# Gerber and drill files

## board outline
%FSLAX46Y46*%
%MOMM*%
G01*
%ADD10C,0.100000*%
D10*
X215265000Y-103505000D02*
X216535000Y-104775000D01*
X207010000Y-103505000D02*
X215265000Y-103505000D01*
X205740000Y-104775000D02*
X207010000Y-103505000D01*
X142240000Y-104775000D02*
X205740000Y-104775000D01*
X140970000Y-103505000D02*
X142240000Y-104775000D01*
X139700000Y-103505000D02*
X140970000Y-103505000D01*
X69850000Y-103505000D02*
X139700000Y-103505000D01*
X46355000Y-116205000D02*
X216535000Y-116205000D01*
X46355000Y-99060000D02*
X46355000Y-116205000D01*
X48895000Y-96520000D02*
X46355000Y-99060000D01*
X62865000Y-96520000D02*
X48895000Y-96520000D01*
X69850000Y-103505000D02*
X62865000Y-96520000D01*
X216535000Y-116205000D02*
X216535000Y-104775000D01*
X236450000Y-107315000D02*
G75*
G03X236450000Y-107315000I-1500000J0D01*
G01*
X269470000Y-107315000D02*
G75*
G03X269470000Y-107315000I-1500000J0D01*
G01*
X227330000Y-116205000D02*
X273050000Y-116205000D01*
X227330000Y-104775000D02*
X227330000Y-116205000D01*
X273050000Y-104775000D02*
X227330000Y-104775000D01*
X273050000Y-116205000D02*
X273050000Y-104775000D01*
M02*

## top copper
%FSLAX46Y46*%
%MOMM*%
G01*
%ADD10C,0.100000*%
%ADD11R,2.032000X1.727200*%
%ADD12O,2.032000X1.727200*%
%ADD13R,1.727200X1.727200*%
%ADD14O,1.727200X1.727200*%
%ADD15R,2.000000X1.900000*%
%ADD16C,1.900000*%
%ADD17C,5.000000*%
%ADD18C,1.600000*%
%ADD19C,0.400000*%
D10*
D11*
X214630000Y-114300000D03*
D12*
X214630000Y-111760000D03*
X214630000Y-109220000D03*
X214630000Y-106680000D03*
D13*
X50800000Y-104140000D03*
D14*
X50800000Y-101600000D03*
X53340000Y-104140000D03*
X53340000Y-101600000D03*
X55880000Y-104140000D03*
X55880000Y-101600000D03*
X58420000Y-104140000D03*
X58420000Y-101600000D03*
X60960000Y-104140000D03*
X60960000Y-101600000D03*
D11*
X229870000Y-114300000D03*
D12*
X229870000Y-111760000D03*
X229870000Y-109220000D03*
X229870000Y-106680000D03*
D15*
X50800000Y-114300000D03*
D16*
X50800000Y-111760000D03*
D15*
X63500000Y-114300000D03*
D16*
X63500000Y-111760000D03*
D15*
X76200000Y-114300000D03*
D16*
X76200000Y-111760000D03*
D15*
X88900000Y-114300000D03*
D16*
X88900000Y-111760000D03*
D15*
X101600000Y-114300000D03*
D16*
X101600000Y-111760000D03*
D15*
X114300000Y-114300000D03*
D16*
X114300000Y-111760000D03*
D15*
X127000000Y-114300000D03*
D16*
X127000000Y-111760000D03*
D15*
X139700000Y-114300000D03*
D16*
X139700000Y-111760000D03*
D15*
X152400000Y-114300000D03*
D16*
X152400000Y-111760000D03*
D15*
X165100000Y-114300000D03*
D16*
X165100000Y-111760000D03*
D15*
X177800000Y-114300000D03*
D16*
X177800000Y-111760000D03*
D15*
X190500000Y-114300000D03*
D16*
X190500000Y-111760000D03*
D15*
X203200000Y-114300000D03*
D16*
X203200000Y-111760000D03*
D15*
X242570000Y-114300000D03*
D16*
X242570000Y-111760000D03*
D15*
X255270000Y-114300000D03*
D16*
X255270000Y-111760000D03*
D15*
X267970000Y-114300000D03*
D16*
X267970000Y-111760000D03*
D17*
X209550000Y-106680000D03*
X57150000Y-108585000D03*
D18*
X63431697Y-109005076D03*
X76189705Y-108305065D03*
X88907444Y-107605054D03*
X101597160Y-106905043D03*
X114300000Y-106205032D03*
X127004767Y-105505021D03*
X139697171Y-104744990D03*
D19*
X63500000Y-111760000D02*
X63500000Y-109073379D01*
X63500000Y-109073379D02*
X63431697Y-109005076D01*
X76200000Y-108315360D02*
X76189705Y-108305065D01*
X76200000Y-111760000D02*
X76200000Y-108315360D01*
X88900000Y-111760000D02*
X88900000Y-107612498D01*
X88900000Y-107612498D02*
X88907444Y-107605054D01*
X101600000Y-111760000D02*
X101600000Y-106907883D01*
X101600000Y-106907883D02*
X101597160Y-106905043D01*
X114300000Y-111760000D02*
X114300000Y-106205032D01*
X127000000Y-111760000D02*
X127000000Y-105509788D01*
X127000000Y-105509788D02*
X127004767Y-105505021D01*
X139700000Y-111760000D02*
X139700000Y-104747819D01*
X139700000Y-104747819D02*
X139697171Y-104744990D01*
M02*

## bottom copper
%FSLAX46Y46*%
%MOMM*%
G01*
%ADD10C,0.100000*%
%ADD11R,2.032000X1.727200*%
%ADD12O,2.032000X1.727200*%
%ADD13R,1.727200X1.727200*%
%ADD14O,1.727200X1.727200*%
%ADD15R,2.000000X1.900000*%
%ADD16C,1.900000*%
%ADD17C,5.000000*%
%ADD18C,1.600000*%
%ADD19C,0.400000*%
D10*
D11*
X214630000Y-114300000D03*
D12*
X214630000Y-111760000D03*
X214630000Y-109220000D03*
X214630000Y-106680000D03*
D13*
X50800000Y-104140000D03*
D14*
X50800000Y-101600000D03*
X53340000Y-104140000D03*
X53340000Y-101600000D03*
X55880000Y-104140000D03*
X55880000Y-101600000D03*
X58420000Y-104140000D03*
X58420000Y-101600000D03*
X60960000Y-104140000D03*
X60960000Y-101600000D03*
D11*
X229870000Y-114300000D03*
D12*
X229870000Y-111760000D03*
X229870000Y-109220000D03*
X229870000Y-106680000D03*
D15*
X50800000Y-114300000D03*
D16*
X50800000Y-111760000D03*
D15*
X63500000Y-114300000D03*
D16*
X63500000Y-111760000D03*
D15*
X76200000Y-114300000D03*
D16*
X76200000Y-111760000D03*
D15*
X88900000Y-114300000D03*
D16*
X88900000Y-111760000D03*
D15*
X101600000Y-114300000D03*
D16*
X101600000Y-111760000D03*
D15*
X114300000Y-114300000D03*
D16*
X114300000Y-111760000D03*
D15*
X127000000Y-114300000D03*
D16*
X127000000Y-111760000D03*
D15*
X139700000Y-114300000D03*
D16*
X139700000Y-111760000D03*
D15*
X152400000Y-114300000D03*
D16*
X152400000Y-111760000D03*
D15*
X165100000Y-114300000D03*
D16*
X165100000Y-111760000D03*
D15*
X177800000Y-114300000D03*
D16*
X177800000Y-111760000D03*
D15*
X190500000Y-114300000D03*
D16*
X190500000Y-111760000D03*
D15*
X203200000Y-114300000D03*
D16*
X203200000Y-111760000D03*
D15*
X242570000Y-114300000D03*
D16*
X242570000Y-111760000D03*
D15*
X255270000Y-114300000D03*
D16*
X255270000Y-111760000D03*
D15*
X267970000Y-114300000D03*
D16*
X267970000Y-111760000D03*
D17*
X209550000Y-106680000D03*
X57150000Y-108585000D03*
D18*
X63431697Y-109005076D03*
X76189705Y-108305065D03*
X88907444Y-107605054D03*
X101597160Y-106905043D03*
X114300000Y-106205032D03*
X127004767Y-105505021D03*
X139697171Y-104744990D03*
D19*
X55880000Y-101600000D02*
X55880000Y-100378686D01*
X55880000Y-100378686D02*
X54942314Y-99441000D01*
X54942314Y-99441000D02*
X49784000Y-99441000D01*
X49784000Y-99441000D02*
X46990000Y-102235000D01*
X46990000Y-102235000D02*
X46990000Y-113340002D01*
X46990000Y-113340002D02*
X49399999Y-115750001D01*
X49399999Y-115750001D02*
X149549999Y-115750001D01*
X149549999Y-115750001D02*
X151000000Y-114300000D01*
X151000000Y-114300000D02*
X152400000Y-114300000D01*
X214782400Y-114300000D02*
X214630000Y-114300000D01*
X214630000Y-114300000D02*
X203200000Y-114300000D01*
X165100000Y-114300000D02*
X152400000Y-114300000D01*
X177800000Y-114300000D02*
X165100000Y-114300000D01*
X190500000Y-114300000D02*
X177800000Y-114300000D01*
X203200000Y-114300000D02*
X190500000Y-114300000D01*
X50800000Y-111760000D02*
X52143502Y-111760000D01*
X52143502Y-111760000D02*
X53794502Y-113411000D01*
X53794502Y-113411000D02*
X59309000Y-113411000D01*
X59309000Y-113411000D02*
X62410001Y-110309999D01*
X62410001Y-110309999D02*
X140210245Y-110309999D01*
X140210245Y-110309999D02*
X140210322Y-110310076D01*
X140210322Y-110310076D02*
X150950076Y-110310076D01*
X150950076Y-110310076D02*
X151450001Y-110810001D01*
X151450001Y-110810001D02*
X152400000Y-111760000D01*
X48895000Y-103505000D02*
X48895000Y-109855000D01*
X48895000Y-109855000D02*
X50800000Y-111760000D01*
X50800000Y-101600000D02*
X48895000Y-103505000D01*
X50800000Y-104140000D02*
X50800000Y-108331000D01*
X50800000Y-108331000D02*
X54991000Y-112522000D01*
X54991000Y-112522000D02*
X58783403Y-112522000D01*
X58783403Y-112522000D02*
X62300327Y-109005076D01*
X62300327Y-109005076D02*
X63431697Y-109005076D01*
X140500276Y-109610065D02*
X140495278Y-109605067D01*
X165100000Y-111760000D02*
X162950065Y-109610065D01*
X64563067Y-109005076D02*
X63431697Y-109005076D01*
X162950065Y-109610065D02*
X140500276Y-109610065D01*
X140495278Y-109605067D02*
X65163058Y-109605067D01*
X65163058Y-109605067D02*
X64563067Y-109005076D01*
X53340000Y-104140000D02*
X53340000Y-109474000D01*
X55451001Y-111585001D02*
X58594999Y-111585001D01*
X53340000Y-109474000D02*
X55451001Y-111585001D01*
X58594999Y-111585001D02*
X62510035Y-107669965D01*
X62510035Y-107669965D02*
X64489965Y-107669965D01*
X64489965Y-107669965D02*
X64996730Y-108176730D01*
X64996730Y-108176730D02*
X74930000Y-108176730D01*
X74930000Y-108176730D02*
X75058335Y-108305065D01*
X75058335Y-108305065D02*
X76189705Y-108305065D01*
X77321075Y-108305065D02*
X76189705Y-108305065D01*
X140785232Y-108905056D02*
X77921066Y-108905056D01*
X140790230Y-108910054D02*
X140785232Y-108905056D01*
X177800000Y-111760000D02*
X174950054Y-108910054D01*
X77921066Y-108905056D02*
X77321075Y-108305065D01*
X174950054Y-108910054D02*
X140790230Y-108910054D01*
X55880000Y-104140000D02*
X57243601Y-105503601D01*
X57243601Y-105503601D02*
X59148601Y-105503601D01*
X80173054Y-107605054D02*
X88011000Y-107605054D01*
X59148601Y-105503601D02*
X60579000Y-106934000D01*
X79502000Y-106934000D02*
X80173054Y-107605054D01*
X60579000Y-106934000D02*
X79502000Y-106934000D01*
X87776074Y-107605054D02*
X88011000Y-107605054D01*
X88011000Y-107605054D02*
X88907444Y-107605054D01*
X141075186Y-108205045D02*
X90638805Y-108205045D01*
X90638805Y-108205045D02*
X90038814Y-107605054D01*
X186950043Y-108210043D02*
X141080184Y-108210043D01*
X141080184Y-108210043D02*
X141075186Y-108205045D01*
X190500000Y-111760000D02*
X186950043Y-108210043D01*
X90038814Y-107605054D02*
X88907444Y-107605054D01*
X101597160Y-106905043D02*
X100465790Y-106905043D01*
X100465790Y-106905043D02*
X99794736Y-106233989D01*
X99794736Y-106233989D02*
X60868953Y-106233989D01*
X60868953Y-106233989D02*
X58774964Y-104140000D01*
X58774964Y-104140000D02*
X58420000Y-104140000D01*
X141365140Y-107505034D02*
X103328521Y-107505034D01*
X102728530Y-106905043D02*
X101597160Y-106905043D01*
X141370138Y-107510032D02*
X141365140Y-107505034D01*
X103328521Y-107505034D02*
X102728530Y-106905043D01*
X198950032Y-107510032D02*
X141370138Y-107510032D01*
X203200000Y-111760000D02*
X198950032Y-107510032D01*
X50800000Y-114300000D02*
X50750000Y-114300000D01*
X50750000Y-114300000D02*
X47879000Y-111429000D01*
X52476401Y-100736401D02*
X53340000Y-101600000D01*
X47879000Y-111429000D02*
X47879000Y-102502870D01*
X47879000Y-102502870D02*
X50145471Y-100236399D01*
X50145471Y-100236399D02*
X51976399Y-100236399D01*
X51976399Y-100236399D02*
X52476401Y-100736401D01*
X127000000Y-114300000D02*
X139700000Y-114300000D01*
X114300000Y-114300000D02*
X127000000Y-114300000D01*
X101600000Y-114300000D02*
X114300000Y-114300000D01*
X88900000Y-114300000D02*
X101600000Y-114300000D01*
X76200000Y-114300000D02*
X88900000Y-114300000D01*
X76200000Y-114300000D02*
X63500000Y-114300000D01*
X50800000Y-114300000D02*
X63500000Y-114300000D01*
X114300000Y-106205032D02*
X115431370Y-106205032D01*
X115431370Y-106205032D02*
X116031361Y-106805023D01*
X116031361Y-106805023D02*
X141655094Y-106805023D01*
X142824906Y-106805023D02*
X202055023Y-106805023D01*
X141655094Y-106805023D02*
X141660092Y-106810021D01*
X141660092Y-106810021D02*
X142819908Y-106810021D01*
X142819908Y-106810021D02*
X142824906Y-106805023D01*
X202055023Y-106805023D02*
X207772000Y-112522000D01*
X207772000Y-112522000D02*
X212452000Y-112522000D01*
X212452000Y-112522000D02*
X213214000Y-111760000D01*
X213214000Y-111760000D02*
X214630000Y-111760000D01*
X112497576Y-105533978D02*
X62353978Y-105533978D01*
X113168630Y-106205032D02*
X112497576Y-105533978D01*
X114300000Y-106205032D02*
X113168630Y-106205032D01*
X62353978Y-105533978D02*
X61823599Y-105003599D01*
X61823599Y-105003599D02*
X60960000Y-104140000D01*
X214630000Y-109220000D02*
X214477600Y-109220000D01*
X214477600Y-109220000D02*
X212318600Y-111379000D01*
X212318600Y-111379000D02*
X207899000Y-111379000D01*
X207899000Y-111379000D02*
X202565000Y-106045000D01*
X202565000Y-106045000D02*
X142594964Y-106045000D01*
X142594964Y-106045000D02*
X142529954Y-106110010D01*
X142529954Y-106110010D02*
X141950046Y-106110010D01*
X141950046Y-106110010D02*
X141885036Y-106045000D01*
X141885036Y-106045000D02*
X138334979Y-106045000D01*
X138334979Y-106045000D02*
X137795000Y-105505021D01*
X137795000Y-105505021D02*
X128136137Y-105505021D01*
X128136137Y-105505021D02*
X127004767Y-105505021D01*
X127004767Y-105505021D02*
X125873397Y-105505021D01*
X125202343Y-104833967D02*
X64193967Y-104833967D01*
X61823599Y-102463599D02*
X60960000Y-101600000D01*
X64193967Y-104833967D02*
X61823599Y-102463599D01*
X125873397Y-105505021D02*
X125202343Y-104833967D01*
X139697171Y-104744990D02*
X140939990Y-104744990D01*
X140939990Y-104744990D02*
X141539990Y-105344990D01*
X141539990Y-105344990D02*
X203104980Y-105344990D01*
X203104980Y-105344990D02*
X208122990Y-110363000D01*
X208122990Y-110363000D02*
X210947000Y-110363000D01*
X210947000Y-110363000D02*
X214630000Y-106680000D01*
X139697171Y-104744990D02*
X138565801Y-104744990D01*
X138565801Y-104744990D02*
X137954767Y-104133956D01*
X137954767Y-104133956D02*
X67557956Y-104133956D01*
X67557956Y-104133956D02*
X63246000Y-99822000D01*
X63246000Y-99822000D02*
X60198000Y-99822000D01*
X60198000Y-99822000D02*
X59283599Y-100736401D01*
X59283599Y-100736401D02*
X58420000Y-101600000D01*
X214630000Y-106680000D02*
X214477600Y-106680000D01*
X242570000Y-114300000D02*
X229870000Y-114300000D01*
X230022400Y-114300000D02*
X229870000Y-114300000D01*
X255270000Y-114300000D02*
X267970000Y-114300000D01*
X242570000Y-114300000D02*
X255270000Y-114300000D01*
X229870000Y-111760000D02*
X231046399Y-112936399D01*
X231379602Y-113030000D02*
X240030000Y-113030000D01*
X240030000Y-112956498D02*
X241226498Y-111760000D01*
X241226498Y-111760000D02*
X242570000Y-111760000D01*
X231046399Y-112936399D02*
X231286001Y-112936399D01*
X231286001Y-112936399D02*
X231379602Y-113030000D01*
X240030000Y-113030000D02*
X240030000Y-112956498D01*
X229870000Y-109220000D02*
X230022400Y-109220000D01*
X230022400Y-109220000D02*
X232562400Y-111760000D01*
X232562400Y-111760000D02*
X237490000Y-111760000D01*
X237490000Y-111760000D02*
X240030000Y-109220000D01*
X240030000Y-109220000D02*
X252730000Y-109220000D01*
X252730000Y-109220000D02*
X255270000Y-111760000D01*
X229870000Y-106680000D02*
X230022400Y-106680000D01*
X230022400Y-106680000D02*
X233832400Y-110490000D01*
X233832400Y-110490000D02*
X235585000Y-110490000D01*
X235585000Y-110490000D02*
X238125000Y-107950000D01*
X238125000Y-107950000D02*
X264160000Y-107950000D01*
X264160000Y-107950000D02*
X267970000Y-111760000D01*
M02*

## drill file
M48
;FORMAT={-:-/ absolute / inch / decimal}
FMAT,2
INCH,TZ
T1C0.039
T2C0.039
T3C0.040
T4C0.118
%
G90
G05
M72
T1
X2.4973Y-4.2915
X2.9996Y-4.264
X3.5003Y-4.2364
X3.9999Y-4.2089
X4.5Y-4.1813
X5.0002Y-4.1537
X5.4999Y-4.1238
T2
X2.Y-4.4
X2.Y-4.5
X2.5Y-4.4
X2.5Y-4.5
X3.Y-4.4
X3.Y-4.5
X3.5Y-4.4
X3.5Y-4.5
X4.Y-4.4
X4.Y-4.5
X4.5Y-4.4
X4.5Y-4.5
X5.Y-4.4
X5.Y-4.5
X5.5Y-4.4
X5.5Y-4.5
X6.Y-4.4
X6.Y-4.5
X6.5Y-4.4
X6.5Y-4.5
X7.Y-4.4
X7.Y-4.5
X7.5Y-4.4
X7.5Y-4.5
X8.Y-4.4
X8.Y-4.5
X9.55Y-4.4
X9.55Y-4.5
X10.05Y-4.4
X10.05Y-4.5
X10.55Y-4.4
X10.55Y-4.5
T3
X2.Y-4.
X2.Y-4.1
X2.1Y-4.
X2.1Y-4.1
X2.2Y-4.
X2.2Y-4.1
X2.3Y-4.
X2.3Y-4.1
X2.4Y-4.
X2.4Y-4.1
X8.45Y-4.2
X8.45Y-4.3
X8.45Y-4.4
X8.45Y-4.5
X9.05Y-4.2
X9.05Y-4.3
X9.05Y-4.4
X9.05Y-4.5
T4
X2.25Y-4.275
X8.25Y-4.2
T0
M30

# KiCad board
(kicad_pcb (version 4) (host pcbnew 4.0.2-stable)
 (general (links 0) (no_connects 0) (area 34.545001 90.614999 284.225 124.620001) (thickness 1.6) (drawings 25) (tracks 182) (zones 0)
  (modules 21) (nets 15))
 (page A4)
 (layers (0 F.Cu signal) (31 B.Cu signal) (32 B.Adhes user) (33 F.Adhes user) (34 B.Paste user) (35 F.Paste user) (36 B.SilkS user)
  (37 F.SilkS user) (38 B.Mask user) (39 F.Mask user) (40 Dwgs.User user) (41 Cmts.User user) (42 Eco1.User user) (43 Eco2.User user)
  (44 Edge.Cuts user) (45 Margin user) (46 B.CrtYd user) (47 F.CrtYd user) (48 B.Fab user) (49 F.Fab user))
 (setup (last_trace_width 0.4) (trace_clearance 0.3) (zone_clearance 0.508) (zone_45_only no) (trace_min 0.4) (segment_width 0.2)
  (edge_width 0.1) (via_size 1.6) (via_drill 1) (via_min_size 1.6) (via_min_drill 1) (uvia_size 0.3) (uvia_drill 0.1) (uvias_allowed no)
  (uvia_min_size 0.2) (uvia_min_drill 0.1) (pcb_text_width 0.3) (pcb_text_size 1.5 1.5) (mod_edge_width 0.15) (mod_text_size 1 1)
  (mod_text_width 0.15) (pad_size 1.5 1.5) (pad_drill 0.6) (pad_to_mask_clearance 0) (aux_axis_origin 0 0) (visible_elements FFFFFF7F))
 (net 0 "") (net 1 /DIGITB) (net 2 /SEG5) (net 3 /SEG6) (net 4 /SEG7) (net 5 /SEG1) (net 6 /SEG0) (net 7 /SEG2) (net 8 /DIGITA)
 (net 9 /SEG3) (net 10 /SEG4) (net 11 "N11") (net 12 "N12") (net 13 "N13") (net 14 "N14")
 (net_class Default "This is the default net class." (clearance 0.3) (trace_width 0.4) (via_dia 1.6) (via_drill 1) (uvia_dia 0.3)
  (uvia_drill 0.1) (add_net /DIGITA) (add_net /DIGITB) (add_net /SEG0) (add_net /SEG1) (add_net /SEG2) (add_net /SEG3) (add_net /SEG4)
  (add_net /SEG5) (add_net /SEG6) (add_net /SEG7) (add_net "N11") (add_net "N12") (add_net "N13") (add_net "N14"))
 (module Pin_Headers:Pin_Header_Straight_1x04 (layer F.Cu) (at 214.63 114.3 180)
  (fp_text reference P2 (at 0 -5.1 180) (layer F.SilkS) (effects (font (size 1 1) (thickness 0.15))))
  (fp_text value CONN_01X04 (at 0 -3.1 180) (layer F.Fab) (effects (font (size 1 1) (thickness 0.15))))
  (pad 1 thru_hole rect (at 0 0 180) (size 2.032 1.7272) (drill 1.016) (layers *.Cu *.Mask F.SilkS) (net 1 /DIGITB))
  (pad 2 thru_hole oval (at 0 2.54 180) (size 2.032 1.7272) (drill 1.016) (layers *.Cu *.Mask F.SilkS) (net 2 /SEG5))
  (pad 3 thru_hole oval (at 0 5.08 180) (size 2.032 1.7272) (drill 1.016) (layers *.Cu *.Mask F.SilkS) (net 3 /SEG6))
  (pad 4 thru_hole oval (at 0 7.62 180) (size 2.032 1.7272) (drill 1.016) (layers *.Cu *.Mask F.SilkS) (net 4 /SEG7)))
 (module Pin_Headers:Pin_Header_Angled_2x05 (layer F.Cu) (at 50.8 104.14 90)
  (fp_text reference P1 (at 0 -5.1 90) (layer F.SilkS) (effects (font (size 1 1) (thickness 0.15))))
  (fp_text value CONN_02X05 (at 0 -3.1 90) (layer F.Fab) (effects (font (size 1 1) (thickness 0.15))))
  (pad 1 thru_hole rect (at 0 0 90) (size 1.7272 1.7272) (drill 1.016) (layers *.Cu *.Mask F.SilkS) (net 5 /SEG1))
  (pad 2 thru_hole oval (at 2.54 0 90) (size 1.7272 1.7272) (drill 1.016) (layers *.Cu *.Mask F.SilkS) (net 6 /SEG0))
  (pad 3 thru_hole oval (at 0 2.54 90) (size 1.7272 1.7272) (drill 1.016) (layers *.Cu *.Mask F.SilkS) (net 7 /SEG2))
  (pad 4 thru_hole oval (at 2.54 2.54 90) (size 1.7272 1.7272) (drill 1.016) (layers *.Cu *.Mask F.SilkS) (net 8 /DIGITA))
  (pad 5 thru_hole oval (at 0 5.08 90) (size 1.7272 1.7272) (drill 1.016) (layers *.Cu *.Mask F.SilkS) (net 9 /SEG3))
  (pad 6 thru_hole oval (at 2.54 5.08 90) (size 1.7272 1.7272) (drill 1.016) (layers *.Cu *.Mask F.SilkS) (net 1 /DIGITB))
  (pad 7 thru_hole oval (at 0 7.62 90) (size 1.7272 1.7272) (drill 1.016) (layers *.Cu *.Mask F.SilkS) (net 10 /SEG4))
  (pad 8 thru_hole oval (at 2.54 7.62 90) (size 1.7272 1.7272) (drill 1.016) (layers *.Cu *.Mask F.SilkS) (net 4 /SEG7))
  (pad 9 thru_hole oval (at 0 10.16 90) (size 1.7272 1.7272) (drill 1.016) (layers *.Cu *.Mask F.SilkS) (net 2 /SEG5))
  (pad 10 thru_hole oval (at 2.54 10.16 90) (size 1.7272 1.7272) (drill 1.016) (layers *.Cu *.Mask F.SilkS) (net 3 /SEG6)))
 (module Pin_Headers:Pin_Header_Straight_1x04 (layer F.Cu) (at 229.87 114.3 180)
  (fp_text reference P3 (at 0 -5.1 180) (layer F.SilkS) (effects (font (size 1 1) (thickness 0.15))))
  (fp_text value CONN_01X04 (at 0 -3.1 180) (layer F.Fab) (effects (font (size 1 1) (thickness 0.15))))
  (pad 1 thru_hole rect (at 0 0 180) (size 2.032 1.7272) (drill 1.016) (layers *.Cu *.Mask F.SilkS) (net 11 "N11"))
  (pad 2 thru_hole oval (at 0 2.54 180) (size 2.032 1.7272) (drill 1.016) (layers *.Cu *.Mask F.SilkS) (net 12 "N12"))
  (pad 3 thru_hole oval (at 0 5.08 180) (size 2.032 1.7272) (drill 1.016) (layers *.Cu *.Mask F.SilkS) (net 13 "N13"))
  (pad 4 thru_hole oval (at 0 7.62 180) (size 2.032 1.7272) (drill 1.016) (layers *.Cu *.Mask F.SilkS) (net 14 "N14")))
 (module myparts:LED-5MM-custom (layer F.Cu) (at 50.8 114.3 90)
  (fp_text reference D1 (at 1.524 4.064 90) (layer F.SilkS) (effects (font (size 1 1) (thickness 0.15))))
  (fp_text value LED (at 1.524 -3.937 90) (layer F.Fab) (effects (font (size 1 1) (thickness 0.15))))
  (pad 1 thru_hole rect (at 0 0 180) (size 2 1.9) (drill 1.00076) (layers *.Cu *.Mask F.SilkS) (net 8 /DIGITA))
  (pad 2 thru_hole circle (at 2.54 0 90) (size 1.9 1.9) (drill 1.00076) (layers *.Cu *.Mask F.SilkS) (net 6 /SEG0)))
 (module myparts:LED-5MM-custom (layer F.Cu) (at 63.5 114.3 90)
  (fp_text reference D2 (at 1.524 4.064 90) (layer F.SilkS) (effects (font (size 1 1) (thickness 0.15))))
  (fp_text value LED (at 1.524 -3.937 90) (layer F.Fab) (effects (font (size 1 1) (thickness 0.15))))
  (pad 1 thru_hole rect (at 0 0 180) (size 2 1.9) (drill 1.00076) (layers *.Cu *.Mask F.SilkS) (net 8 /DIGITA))
  (pad 2 thru_hole circle (at 2.54 0 90) (size 1.9 1.9) (drill 1.00076) (layers *.Cu *.Mask F.SilkS) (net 5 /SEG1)))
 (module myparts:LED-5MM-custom (layer F.Cu) (at 76.2 114.3 90)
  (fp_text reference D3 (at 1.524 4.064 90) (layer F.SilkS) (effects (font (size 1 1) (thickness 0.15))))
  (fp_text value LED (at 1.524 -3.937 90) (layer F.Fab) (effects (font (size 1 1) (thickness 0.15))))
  (pad 1 thru_hole rect (at 0 0 180) (size 2 1.9) (drill 1.00076) (layers *.Cu *.Mask F.SilkS) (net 8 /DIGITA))
  (pad 2 thru_hole circle (at 2.54 0 90) (size 1.9 1.9) (drill 1.00076) (layers *.Cu *.Mask F.SilkS) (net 7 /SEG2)))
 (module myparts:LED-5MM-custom (layer F.Cu) (at 88.9 114.3 90)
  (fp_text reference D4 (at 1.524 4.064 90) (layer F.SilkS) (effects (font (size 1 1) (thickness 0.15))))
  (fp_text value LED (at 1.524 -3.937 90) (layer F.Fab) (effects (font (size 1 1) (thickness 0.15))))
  (pad 1 thru_hole rect (at 0 0 180) (size 2 1.9) (drill 1.00076) (layers *.Cu *.Mask F.SilkS) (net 8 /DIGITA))
  (pad 2 thru_hole circle (at 2.54 0 90) (size 1.9 1.9) (drill 1.00076) (layers *.Cu *.Mask F.SilkS) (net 9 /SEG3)))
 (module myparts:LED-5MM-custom (layer F.Cu) (at 101.6 114.3 90)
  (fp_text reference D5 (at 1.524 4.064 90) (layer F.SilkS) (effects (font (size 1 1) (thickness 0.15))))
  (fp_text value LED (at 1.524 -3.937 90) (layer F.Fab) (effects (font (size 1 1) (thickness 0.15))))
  (pad 1 thru_hole rect (at 0 0 180) (size 2 1.9) (drill 1.00076) (layers *.Cu *.Mask F.SilkS) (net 8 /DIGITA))
  (pad 2 thru_hole circle (at 2.54 0 90) (size 1.9 1.9) (drill 1.00076) (layers *.Cu *.Mask F.SilkS) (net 10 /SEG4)))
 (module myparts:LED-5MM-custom (layer F.Cu) (at 114.3 114.3 90)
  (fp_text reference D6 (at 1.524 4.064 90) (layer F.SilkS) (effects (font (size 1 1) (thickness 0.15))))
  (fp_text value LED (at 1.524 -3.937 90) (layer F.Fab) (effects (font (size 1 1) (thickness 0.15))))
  (pad 1 thru_hole rect (at 0 0 180) (size 2 1.9) (drill 1.00076) (layers *.Cu *.Mask F.SilkS) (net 8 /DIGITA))
  (pad 2 thru_hole circle (at 2.54 0 90) (size 1.9 1.9) (drill 1.00076) (layers *.Cu *.Mask F.SilkS) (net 2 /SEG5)))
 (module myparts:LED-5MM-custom (layer F.Cu) (at 127 114.3 90)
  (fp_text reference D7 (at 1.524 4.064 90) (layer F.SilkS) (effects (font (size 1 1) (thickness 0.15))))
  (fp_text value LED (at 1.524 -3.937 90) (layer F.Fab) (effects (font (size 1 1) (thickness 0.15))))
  (pad 1 thru_hole rect (at 0 0 180) (size 2 1.9) (drill 1.00076) (layers *.Cu *.Mask F.SilkS) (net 8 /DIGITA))
  (pad 2 thru_hole circle (at 2.54 0 90) (size 1.9 1.9) (drill 1.00076) (layers *.Cu *.Mask F.SilkS) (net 3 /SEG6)))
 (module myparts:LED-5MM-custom (layer F.Cu) (at 139.7 114.3 90)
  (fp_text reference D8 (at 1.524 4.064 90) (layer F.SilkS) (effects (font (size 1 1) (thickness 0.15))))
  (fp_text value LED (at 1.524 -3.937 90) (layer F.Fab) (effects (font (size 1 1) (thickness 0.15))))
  (pad 1 thru_hole rect (at 0 0 180) (size 2 1.9) (drill 1.00076) (layers *.Cu *.Mask F.SilkS) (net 8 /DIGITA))
  (pad 2 thru_hole circle (at 2.54 0 90) (size 1.9 1.9) (drill 1.00076) (layers *.Cu *.Mask F.SilkS) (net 4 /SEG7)))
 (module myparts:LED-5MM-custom (layer F.Cu) (at 152.4 114.3 90)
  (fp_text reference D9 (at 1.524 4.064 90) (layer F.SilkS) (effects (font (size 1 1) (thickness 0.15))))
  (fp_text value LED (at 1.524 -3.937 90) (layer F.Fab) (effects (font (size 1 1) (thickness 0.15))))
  (pad 1 thru_hole rect (at 0 0 180) (size 2 1.9) (drill 1.00076) (layers *.Cu *.Mask F.SilkS) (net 1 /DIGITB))
  (pad 2 thru_hole circle (at 2.54 0 90) (size 1.9 1.9) (drill 1.00076) (layers *.Cu *.Mask F.SilkS) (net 6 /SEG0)))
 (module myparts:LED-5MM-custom (layer F.Cu) (at 165.1 114.3 90)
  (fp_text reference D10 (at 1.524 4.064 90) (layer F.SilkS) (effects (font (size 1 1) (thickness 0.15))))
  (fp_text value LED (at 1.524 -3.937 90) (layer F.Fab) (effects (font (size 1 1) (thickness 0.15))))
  (pad 1 thru_hole rect (at 0 0 180) (size 2 1.9) (drill 1.00076) (layers *.Cu *.Mask F.SilkS) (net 1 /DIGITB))
  (pad 2 thru_hole circle (at 2.54 0 90) (size 1.9 1.9) (drill 1.00076) (layers *.Cu *.Mask F.SilkS) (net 5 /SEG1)))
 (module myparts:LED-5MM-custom (layer F.Cu) (at 177.8 114.3 90)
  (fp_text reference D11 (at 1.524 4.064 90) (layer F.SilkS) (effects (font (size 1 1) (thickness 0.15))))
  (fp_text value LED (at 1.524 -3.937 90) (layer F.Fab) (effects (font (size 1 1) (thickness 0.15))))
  (pad 1 thru_hole rect (at 0 0 180) (size 2 1.9) (drill 1.00076) (layers *.Cu *.Mask F.SilkS) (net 1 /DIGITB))
  (pad 2 thru_hole circle (at 2.54 0 90) (size 1.9 1.9) (drill 1.00076) (layers *.Cu *.Mask F.SilkS) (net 7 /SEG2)))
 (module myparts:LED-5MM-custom (layer F.Cu) (at 190.5 114.3 90)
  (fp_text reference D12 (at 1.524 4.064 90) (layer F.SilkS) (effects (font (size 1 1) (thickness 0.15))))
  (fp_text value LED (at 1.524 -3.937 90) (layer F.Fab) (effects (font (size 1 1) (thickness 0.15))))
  (pad 1 thru_hole rect (at 0 0 180) (size 2 1.9) (drill 1.00076) (layers *.Cu *.Mask F.SilkS) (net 1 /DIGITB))
  (pad 2 thru_hole circle (at 2.54 0 90) (size 1.9 1.9) (drill 1.00076) (layers *.Cu *.Mask F.SilkS) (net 9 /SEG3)))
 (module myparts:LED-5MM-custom (layer F.Cu) (at 203.2 114.3 90)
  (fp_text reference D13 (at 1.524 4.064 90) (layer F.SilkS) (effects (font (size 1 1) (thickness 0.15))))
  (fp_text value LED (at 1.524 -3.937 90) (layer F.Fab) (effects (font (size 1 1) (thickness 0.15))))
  (pad 1 thru_hole rect (at 0 0 180) (size 2 1.9) (drill 1.00076) (layers *.Cu *.Mask F.SilkS) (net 1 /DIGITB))
  (pad 2 thru_hole circle (at 2.54 0 90) (size 1.9 1.9) (drill 1.00076) (layers *.Cu *.Mask F.SilkS) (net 10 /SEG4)))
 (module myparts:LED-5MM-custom (layer F.Cu) (at 242.57 114.3 90)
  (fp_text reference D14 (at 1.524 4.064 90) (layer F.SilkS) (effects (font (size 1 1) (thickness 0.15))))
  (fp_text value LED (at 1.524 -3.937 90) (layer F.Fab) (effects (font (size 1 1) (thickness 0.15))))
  (pad 1 thru_hole rect (at 0 0 180) (size 2 1.9) (drill 1.00076) (layers *.Cu *.Mask F.SilkS) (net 11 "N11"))
  (pad 2 thru_hole circle (at 2.54 0 90) (size 1.9 1.9) (drill 1.00076) (layers *.Cu *.Mask F.SilkS) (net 12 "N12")))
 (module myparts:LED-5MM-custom (layer F.Cu) (at 255.27 114.3 90)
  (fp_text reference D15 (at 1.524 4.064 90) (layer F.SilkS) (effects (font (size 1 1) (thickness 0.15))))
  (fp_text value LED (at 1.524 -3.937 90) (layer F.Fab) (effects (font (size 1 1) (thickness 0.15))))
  (pad 1 thru_hole rect (at 0 0 180) (size 2 1.9) (drill 1.00076) (layers *.Cu *.Mask F.SilkS) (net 11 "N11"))
  (pad 2 thru_hole circle (at 2.54 0 90) (size 1.9 1.9) (drill 1.00076) (layers *.Cu *.Mask F.SilkS) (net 13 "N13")))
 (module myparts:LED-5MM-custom (layer F.Cu) (at 267.97 114.3 90)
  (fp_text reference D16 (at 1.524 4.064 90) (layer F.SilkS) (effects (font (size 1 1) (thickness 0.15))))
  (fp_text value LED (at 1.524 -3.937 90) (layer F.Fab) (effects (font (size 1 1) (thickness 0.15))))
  (pad 1 thru_hole rect (at 0 0 180) (size 2 1.9) (drill 1.00076) (layers *.Cu *.Mask F.SilkS) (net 11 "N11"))
  (pad 2 thru_hole circle (at 2.54 0 90) (size 1.9 1.9) (drill 1.00076) (layers *.Cu *.Mask F.SilkS) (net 14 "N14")))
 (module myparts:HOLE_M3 (layer F.Cu) (at 209.55 106.68)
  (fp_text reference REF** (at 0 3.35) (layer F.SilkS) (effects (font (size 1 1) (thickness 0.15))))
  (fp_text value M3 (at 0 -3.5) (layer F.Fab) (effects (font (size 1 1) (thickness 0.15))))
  (pad 1 thru_hole circle (at 0 0) (size 5 5) (drill 3) (layers *.Cu *.Mask F.SilkS)))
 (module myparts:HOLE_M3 (layer F.Cu) (at 57.15 108.585)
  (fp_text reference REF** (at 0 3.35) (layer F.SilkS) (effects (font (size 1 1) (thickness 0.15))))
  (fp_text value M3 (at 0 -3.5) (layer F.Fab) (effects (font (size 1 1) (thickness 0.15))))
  (pad 1 thru_hole circle (at 0 0) (size 5 5) (drill 3) (layers *.Cu *.Mask F.SilkS)))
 (gr_line (start 215.265 103.505) (end 216.535 104.775) (layer Edge.Cuts) (width 0.1))
 (gr_line (start 207.01 103.505) (end 215.265 103.505) (layer Edge.Cuts) (width 0.1))
 (gr_line (start 205.74 104.775) (end 207.01 103.505) (layer Edge.Cuts) (width 0.1))
 (gr_line (start 142.24 104.775) (end 205.74 104.775) (layer Edge.Cuts) (width 0.1))
 (gr_line (start 140.97 103.505) (end 142.24 104.775) (layer Edge.Cuts) (width 0.1))
 (gr_line (start 139.7 103.505) (end 140.97 103.505) (layer Edge.Cuts) (width 0.1))
 (gr_line (start 69.85 103.505) (end 139.7 103.505) (layer Edge.Cuts) (width 0.1))
 (gr_line (start 46.355 116.205) (end 216.535 116.205) (layer Edge.Cuts) (width 0.1))
 (gr_line (start 46.355 99.06) (end 46.355 116.205) (layer Edge.Cuts) (width 0.1))
 (gr_line (start 48.895 96.52) (end 46.355 99.06) (layer Edge.Cuts) (width 0.1))
 (gr_line (start 62.865 96.52) (end 48.895 96.52) (layer Edge.Cuts) (width 0.1))
 (gr_line (start 69.85 103.505) (end 62.865 96.52) (layer Edge.Cuts) (width 0.1))
 (gr_line (start 216.535 116.205) (end 216.535 104.775) (layer Edge.Cuts) (width 0.1))
 (gr_circle (center 234.95 107.315) (end 236.45 107.315) (layer Edge.Cuts) (width 0.1))
 (gr_circle (center 267.97 107.315) (end 269.47 107.315) (layer Edge.Cuts) (width 0.1))
 (gr_line (start 227.33 116.205) (end 273.05 116.205) (layer Edge.Cuts) (width 0.1))
 (gr_line (start 227.33 104.775) (end 227.33 116.205) (layer Edge.Cuts) (width 0.1))
 (gr_line (start 273.05 104.775) (end 227.33 104.775) (layer Edge.Cuts) (width 0.1))
 (gr_line (start 273.05 116.205) (end 273.05 104.775) (layer Edge.Cuts) (width 0.1))
 (segment (start 55.88 101.6) (end 55.88 100.378686) (width 0.4) (layer B.Cu) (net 1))
 (segment (start 55.88 100.378686) (end 54.942314 99.441) (width 0.4) (layer B.Cu) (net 1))
 (segment (start 54.942314 99.441) (end 49.784 99.441) (width 0.4) (layer B.Cu) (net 1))
 (segment (start 49.784 99.441) (end 46.99 102.235) (width 0.4) (layer B.Cu) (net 1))
 (segment (start 46.99 102.235) (end 46.99 113.340002) (width 0.4) (layer B.Cu) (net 1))
 (segment (start 46.99 113.340002) (end 49.399999 115.750001) (width 0.4) (layer B.Cu) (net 1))
 (segment (start 49.399999 115.750001) (end 149.549999 115.750001) (width 0.4) (layer B.Cu) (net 1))
 (segment (start 149.549999 115.750001) (end 151 114.3) (width 0.4) (layer B.Cu) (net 1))
 (segment (start 151 114.3) (end 152.4 114.3) (width 0.4) (layer B.Cu) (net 1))
 (segment (start 214.7824 114.3) (end 214.63 114.3) (width 0.4) (layer B.Cu) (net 1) (status 30))
 (segment (start 214.63 114.3) (end 203.2 114.3) (width 0.4) (layer B.Cu) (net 1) (status 30))
 (segment (start 165.1 114.3) (end 152.4 114.3) (width 0.4) (layer B.Cu) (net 1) (status 30))
 (segment (start 177.8 114.3) (end 165.1 114.3) (width 0.4) (layer B.Cu) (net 1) (status 30))
 (segment (start 190.5 114.3) (end 177.8 114.3) (width 0.4) (layer B.Cu) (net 1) (status 30))
 (segment (start 203.2 114.3) (end 190.5 114.3) (width 0.4) (layer B.Cu) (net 1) (status 30))
 (segment (start 50.8 111.76) (end 52.143502 111.76) (width 0.4) (layer B.Cu) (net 6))
 (segment (start 52.143502 111.76) (end 53.794502 113.411) (width 0.4) (layer B.Cu) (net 6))
 (segment (start 53.794502 113.411) (end 59.309 113.411) (width 0.4) (layer B.Cu) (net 6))
 (segment (start 59.309 113.411) (end 62.410001 110.309999) (width 0.4) (layer B.Cu) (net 6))
 (segment (start 62.410001 110.309999) (end 140.210245 110.309999) (width 0.4) (layer B.Cu) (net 6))
 (segment (start 140.210245 110.309999) (end 140.210322 110.310076) (width 0.4) (layer B.Cu) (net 6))
 (segment (start 140.210322 110.310076) (end 150.950076 110.310076) (width 0.4) (layer B.Cu) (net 6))
 (segment (start 150.950076 110.310076) (end 151.450001 110.810001) (width 0.4) (layer B.Cu) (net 6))
 (segment (start 151.450001 110.810001) (end 152.4 111.76) (width 0.4) (layer B.Cu) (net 6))
 (segment (start 48.895 103.505) (end 48.895 109.855) (width 0.4) (layer B.Cu) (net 6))
 (segment (start 48.895 109.855) (end 50.8 111.76) (width 0.4) (layer B.Cu) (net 6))
 (segment (start 50.8 101.6) (end 48.895 103.505) (width 0.4) (layer B.Cu) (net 6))
 (segment (start 50.8 104.14) (end 50.8 108.331) (width 0.4) (layer B.Cu) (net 5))
 (segment (start 50.8 108.331) (end 54.991 112.522) (width 0.4) (layer B.Cu) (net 5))
 (segment (start 54.991 112.522) (end 58.783403 112.522) (width 0.4) (layer B.Cu) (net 5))
 (segment (start 58.783403 112.522) (end 62.300327 109.005076) (width 0.4) (layer B.Cu) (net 5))
 (segment (start 62.300327 109.005076) (end 63.431697 109.005076) (width 0.4) (layer B.Cu) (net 5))
 (segment (start 140.500276 109.610065) (end 140.495278 109.605067) (width 0.4) (layer B.Cu) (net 5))
 (via (at 63.431697 109.005076) (size 1.6) (drill 1) (layers F.Cu B.Cu) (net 5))
 (segment (start 165.1 111.76) (end 162.950065 109.610065) (width 0.4) (layer B.Cu) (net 5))
 (segment (start 64.563067 109.005076) (end 63.431697 109.005076) (width 0.4) (layer B.Cu) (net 5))
 (segment (start 162.950065 109.610065) (end 140.500276 109.610065) (width 0.4) (layer B.Cu) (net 5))
 (segment (start 140.495278 109.605067) (end 65.163058 109.605067) (width 0.4) (layer B.Cu) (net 5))
 (segment (start 63.5 111.76) (end 63.5 109.073379) (width 0.4) (layer F.Cu) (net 5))
 (segment (start 65.163058 109.605067) (end 64.563067 109.005076) (width 0.4) (layer B.Cu) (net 5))
 (segment (start 63.5 109.073379) (end 63.431697 109.005076) (width 0.4) (layer F.Cu) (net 5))
 (segment (start 53.34 104.14) (end 53.34 109.474) (width 0.4) (layer B.Cu) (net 7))
 (segment (start 55.451001 111.585001) (end 58.594999 111.585001) (width 0.4) (layer B.Cu) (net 7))
 (segment (start 53.34 109.474) (end 55.451001 111.585001) (width 0.4) (layer B.Cu) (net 7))
 (segment (start 58.594999 111.585001) (end 62.510035 107.669965) (width 0.4) (layer B.Cu) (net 7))
 (segment (start 62.510035 107.669965) (end 64.489965 107.669965) (width 0.4) (layer B.Cu) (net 7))
 (segment (start 64.489965 107.669965) (end 64.99673 108.17673) (width 0.4) (layer B.Cu) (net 7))
 (segment (start 64.99673 108.17673) (end 74.93 108.17673) (width 0.4) (layer B.Cu) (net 7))
 (segment (start 74.93 108.17673) (end 75.058335 108.305065) (width 0.4) (layer B.Cu) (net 7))
 (segment (start 75.058335 108.305065) (end 76.189705 108.305065) (width 0.4) (layer B.Cu) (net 7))
 (segment (start 77.321075 108.305065) (end 76.189705 108.305065) (width 0.4) (layer B.Cu) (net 7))
 (segment (start 140.785232 108.905056) (end 77.921066 108.905056) (width 0.4) (layer B.Cu) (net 7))
 (segment (start 140.79023 108.910054) (end 140.785232 108.905056) (width 0.4) (layer B.Cu) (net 7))
 (segment (start 177.8 111.76) (end 174.950054 108.910054) (width 0.4) (layer B.Cu) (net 7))
 (segment (start 77.921066 108.905056) (end 77.321075 108.305065) (width 0.4) (layer B.Cu) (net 7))
 (segment (start 174.950054 108.910054) (end 140.79023 108.910054) (width 0.4) (layer B.Cu) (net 7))
 (segment (start 76.2 108.31536) (end 76.189705 108.305065) (width 0.4) (layer F.Cu) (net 7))
 (segment (start 76.2 111.76) (end 76.2 108.31536) (width 0.4) (layer F.Cu) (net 7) (status 10))
 (via (at 76.189705 108.305065) (size 1.6) (drill 1) (layers F.Cu B.Cu) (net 7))
 (segment (start 55.88 104.14) (end 57.243601 105.503601) (width 0.4) (layer B.Cu) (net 9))
 (segment (start 57.243601 105.503601) (end 59.148601 105.503601) (width 0.4) (layer B.Cu) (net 9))
 (segment (start 80.173054 107.605054) (end 88.011 107.605054) (width 0.4) (layer B.Cu) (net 9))
 (segment (start 59.148601 105.503601) (end 60.579 106.934) (width 0.4) (layer B.Cu) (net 9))
 (segment (start 79.502 106.934) (end 80.173054 107.605054) (width 0.4) (layer B.Cu) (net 9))
 (segment (start 60.579 106.934) (end 79.502 106.934) (width 0.4) (layer B.Cu) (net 9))
 (segment (start 87.776074 107.605054) (end 88.011 107.605054) (width 0.4) (layer B.Cu) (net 9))
 (segment (start 88.011 107.605054) (end 88.907444 107.605054) (width 0.4) (layer B.Cu) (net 9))
 (segment (start 141.075186 108.205045) (end 90.638805 108.205045) (width 0.4) (layer B.Cu) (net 9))
 (segment (start 90.638805 108.205045) (end 90.038814 107.605054) (width 0.4) (layer B.Cu) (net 9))
 (segment (start 186.950043 108.210043) (end 141.080184 108.210043) (width 0.4) (layer B.Cu) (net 9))
 (segment (start 141.080184 108.210043) (end 141.075186 108.205045) (width 0.4) (layer B.Cu) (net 9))
 (segment (start 190.5 111.76) (end 186.950043 108.210043) (width 0.4) (layer B.Cu) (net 9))
 (segment (start 90.038814 107.605054) (end 88.907444 107.605054) (width 0.4) (layer B.Cu) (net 9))
 (via (at 88.907444 107.605054) (size 1.6) (drill 1) (layers F.Cu B.Cu) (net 9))
 (segment (start 88.9 111.76) (end 88.9 107.612498) (width 0.4) (layer F.Cu) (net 9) (status 10))
 (segment (start 88.9 107.612498) (end 88.907444 107.605054) (width 0.4) (layer F.Cu) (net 9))
 (segment (start 101.59716 106.905043) (end 100.46579 106.905043) (width 0.4) (layer B.Cu) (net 10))
 (segment (start 100.46579 106.905043) (end 99.794736 106.233989) (width 0.4) (layer B.Cu) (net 10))
 (segment (start 99.794736 106.233989) (end 60.868953 106.233989) (width 0.4) (layer B.Cu) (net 10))
 (segment (start 60.868953 106.233989) (end 58.774964 104.14) (width 0.4) (layer B.Cu) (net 10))
 (segment (start 58.774964 104.14) (end 58.42 104.14) (width 0.4) (layer B.Cu) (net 10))
 (segment (start 141.36514 107.505034) (end 103.328521 107.505034) (width 0.4) (layer B.Cu) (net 10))
 (segment (start 102.72853 106.905043) (end 101.59716 106.905043) (width 0.4) (layer B.Cu) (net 10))
 (segment (start 141.370138 107.510032) (end 141.36514 107.505034) (width 0.4) (layer B.Cu) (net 10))
 (segment (start 103.328521 107.505034) (end 102.72853 106.905043) (width 0.4) (layer B.Cu) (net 10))
 (segment (start 198.950032 107.510032) (end 141.370138 107.510032) (width 0.4) (layer B.Cu) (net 10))
 (segment (start 203.2 111.76) (end 198.950032 107.510032) (width 0.4) (layer B.Cu) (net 10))
 (segment (start 101.6 111.76) (end 101.6 106.907883) (width 0.4) (layer F.Cu) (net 10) (status 10))
 (via (at 101.59716 106.905043) (size 1.6) (drill 1) (layers F.Cu B.Cu) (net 10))
 (segment (start 101.6 106.907883) (end 101.59716 106.905043) (width 0.4) (layer F.Cu) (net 10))
 (segment (start 50.8 114.3) (end 50.75 114.3) (width 0.4) (layer B.Cu) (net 8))
 (segment (start 50.75 114.3) (end 47.879 111.429) (width 0.4) (layer B.Cu) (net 8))
 (segment (start 52.476401 100.736401) (end 53.34 101.6) (width 0.4) (layer B.Cu) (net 8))
 (segment (start 47.879 111.429) (end 47.879 102.50287) (width 0.4) (layer B.Cu) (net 8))
 (segment (start 47.879 102.50287) (end 50.145471 100.236399) (width 0.4) (layer B.Cu) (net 8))
 (segment (start 50.145471 100.236399) (end 51.976399 100.236399) (width 0.4) (layer B.Cu) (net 8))
 (segment (start 51.976399 100.236399) (end 52.476401 100.736401) (width 0.4) (layer B.Cu) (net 8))
 (segment (start 127 114.3) (end 139.7 114.3) (width 0.4) (layer B.Cu) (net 8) (status 30))
 (segment (start 114.3 114.3) (end 127 114.3) (width 0.4) (layer B.Cu) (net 8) (status 30))
 (segment (start 101.6 114.3) (end 114.3 114.3) (width 0.4) (layer B.Cu) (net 8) (status 30))
 (segment (start 88.9 114.3) (end 101.6 114.3) (width 0.4) (layer B.Cu) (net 8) (status 30))
 (segment (start 76.2 114.3) (end 88.9 114.3) (width 0.4) (layer B.Cu) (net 8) (status 30))
 (segment (start 76.2 114.3) (end 63.5 114.3) (width 0.4) (layer B.Cu) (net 8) (status 30))
 (segment (start 50.8 114.3) (end 63.5 114.3) (width 0.4) (layer B.Cu) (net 8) (status 30))
 (segment (start 114.3 106.205032) (end 115.43137 106.205032) (width 0.4) (layer B.Cu) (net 2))
 (segment (start 115.43137 106.205032) (end 116.031361 106.805023) (width 0.4) (layer B.Cu) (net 2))
 (segment (start 116.031361 106.805023) (end 141.655094 106.805023) (width 0.4) (layer B.Cu) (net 2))
 (segment (start 142.824906 106.805023) (end 202.055023 106.805023) (width 0.4) (layer B.Cu) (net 2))
 (segment (start 141.655094 106.805023) (end 141.660092 106.810021) (width 0.4) (layer B.Cu) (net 2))
 (segment (start 141.660092 106.810021) (end 142.819908 106.810021) (width 0.4) (layer B.Cu) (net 2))
 (segment (start 142.819908 106.810021) (end 142.824906 106.805023) (width 0.4) (layer B.Cu) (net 2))
 (segment (start 202.055023 106.805023) (end 207.772 112.522) (width 0.4) (layer B.Cu) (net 2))
 (segment (start 207.772 112.522) (end 212.452 112.522) (width 0.4) (layer B.Cu) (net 2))
 (segment (start 212.452 112.522) (end 213.214 111.76) (width 0.4) (layer B.Cu) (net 2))
 (segment (start 213.214 111.76) (end 214.63 111.76) (width 0.4) (layer B.Cu) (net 2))
 (segment (start 112.497576 105.533978) (end 62.353978 105.533978) (width 0.4) (layer B.Cu) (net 2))
 (segment (start 113.16863 106.205032) (end 112.497576 105.533978) (width 0.4) (layer B.Cu) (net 2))
 (segment (start 114.3 106.205032) (end 113.16863 106.205032) (width 0.4) (layer B.Cu) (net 2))
 (segment (start 62.353978 105.533978) (end 61.823599 105.003599) (width 0.4) (layer B.Cu) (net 2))
 (segment (start 61.823599 105.003599) (end 60.96 104.14) (width 0.4) (layer B.Cu) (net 2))
 (via (at 114.3 106.205032) (size 1.6) (drill 1) (layers F.Cu B.Cu) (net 2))
 (segment (start 114.3 111.76) (end 114.3 106.205032) (width 0.4) (layer F.Cu) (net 2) (status 10))
 (segment (start 214.63 109.22) (end 214.4776 109.22) (width 0.4) (layer B.Cu) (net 3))
 (segment (start 214.4776 109.22) (end 212.3186 111.379) (width 0.4) (layer B.Cu) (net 3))
 (segment (start 212.3186 111.379) (end 207.899 111.379) (width 0.4) (layer B.Cu) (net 3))
 (segment (start 207.899 111.379) (end 202.565 106.045) (width 0.4) (layer B.Cu) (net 3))
 (segment (start 202.565 106.045) (end 142.594964 106.045) (width 0.4) (layer B.Cu) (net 3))
 (segment (start 142.594964 106.045) (end 142.529954 106.11001) (width 0.4) (layer B.Cu) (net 3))
 (segment (start 142.529954 106.11001) (end 141.950046 106.11001) (width 0.4) (layer B.Cu) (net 3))
 (segment (start 141.950046 106.11001) (end 141.885036 106.045) (width 0.4) (layer B.Cu) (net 3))
 (segment (start 141.885036 106.045) (end 138.334979 106.045) (width 0.4) (layer B.Cu) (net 3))
 (segment (start 138.334979 106.045) (end 137.795 105.505021) (width 0.4) (layer B.Cu) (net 3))
 (segment (start 137.795 105.505021) (end 128.136137 105.505021) (width 0.4) (layer B.Cu) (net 3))
 (segment (start 128.136137 105.505021) (end 127.004767 105.505021) (width 0.4) (layer B.Cu) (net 3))
 (segment (start 127.004767 105.505021) (end 125.873397 105.505021) (width 0.4) (layer B.Cu) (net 3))
 (segment (start 125.202343 104.833967) (end 64.193967 104.833967) (width 0.4) (layer B.Cu) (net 3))
 (segment (start 61.823599 102.463599) (end 60.96 101.6) (width 0.4) (layer B.Cu) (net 3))
 (segment (start 64.193967 104.833967) (end 61.823599 102.463599) (width 0.4) (layer B.Cu) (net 3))
 (segment (start 125.873397 105.505021) (end 125.202343 104.833967) (width 0.4) (layer B.Cu) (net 3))
 (segment (start 127 111.76) (end 127 105.509788) (width 0.4) (layer F.Cu) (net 3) (status 10))
 (via (at 127.004767 105.505021) (size 1.6) (drill 1) (layers F.Cu B.Cu) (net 3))
 (segment (start 127 105.509788) (end 127.004767 105.505021) (width 0.4) (layer F.Cu) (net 3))
 (segment (start 139.697171 104.74499) (end 140.93999 104.74499) (width 0.4) (layer B.Cu) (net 4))
 (segment (start 140.93999 104.74499) (end 141.53999 105.34499) (width 0.4) (layer B.Cu) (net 4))
 (segment (start 141.53999 105.34499) (end 203.10498 105.34499) (width 0.4) (layer B.Cu) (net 4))
 (segment (start 203.10498 105.34499) (end 208.12299 110.363) (width 0.4) (layer B.Cu) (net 4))
 (segment (start 208.12299 110.363) (end 210.947 110.363) (width 0.4) (layer B.Cu) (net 4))
 (segment (start 210.947 110.363) (end 214.63 106.68) (width 0.4) (layer B.Cu) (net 4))
 (segment (start 139.697171 104.74499) (end 138.565801 104.74499) (width 0.4) (layer B.Cu) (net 4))
 (segment (start 138.565801 104.74499) (end 137.954767 104.133956) (width 0.4) (layer B.Cu) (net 4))
 (segment (start 137.954767 104.133956) (end 67.557956 104.133956) (width 0.4) (layer B.Cu) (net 4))
 (segment (start 67.557956 104.133956) (end 63.246 99.822) (width 0.4) (layer B.Cu) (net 4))
 (segment (start 63.246 99.822) (end 60.198 99.822) (width 0.4) (layer B.Cu) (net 4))
 (segment (start 60.198 99.822) (end 59.283599 100.736401) (width 0.4) (layer B.Cu) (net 4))
 (segment (start 59.283599 100.736401) (end 58.42 101.6) (width 0.4) (layer B.Cu) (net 4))
 (segment (start 139.7 111.76) (end 139.7 104.747819) (width 0.4) (layer F.Cu) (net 4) (status 10))
 (segment (start 139.7 104.747819) (end 139.697171 104.74499) (width 0.4) (layer F.Cu) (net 4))
 (via (at 139.697171 104.74499) (size 1.6) (drill 1) (layers F.Cu B.Cu) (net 4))
 (segment (start 214.63 106.68) (end 214.4776 106.68) (width 0.4) (layer B.Cu) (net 4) (status 30))
 (segment (start 242.57 114.3) (end 229.87 114.3) (width 0.4) (layer B.Cu) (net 11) (status 30))
 (segment (start 230.0224 114.3) (end 229.87 114.3) (width 0.4) (layer B.Cu) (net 11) (status 30))
 (segment (start 255.27 114.3) (end 267.97 114.3) (width 0.4) (layer B.Cu) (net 11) (status 30))
 (segment (start 242.57 114.3) (end 255.27 114.3) (width 0.4) (layer B.Cu) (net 11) (status 30))
 (segment (start 229.87 111.76) (end 231.046399 112.936399) (width 0.4) (layer B.Cu) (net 12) (status 10))
 (segment (start 231.379602 113.03) (end 240.03 113.03) (width 0.4) (layer B.Cu) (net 12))
 (segment (start 240.03 112.956498) (end 241.226498 111.76) (width 0.4) (layer B.Cu) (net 12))
 (segment (start 241.226498 111.76) (end 242.57 111.76) (width 0.4) (layer B.Cu) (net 12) (status 20))
 (segment (start 231.046399 112.936399) (end 231.286001 112.936399) (width 0.4) (layer B.Cu) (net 12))
 (segment (start 231.286001 112.936399) (end 231.379602 113.03) (width 0.4) (layer B.Cu) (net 12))
 (segment (start 240.03 113.03) (end 240.03 112.956498) (width 0.4) (layer B.Cu) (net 12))
 (segment (start 229.87 109.22) (end 230.0224 109.22) (width 0.4) (layer B.Cu) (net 13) (status 30))
 (segment (start 230.0224 109.22) (end 232.5624 111.76) (width 0.4) (layer B.Cu) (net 13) (status 10))
 (segment (start 232.5624 111.76) (end 237.49 111.76) (width 0.4) (layer B.Cu) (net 13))
 (segment (start 237.49 111.76) (end 240.03 109.22) (width 0.4) (layer B.Cu) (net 13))
 (segment (start 240.03 109.22) (end 252.73 109.22) (width 0.4) (layer B.Cu) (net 13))
 (segment (start 252.73 109.22) (end 255.27 111.76) (width 0.4) (layer B.Cu) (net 13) (status 20))
 (segment (start 229.87 106.68) (end 230.0224 106.68) (width 0.4) (layer B.Cu) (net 14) (status 30))
 (segment (start 230.0224 106.68) (end 233.8324 110.49) (width 0.4) (layer B.Cu) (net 14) (status 10))
 (segment (start 233.8324 110.49) (end 235.585 110.49) (width 0.4) (layer B.Cu) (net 14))
 (segment (start 235.585 110.49) (end 238.125 107.95) (width 0.4) (layer B.Cu) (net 14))
 (segment (start 238.125 107.95) (end 264.16 107.95) (width 0.4) (layer B.Cu) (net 14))
 (segment (start 264.16 107.95) (end 267.97 111.76) (width 0.4) (layer B.Cu) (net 14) (status 20)))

